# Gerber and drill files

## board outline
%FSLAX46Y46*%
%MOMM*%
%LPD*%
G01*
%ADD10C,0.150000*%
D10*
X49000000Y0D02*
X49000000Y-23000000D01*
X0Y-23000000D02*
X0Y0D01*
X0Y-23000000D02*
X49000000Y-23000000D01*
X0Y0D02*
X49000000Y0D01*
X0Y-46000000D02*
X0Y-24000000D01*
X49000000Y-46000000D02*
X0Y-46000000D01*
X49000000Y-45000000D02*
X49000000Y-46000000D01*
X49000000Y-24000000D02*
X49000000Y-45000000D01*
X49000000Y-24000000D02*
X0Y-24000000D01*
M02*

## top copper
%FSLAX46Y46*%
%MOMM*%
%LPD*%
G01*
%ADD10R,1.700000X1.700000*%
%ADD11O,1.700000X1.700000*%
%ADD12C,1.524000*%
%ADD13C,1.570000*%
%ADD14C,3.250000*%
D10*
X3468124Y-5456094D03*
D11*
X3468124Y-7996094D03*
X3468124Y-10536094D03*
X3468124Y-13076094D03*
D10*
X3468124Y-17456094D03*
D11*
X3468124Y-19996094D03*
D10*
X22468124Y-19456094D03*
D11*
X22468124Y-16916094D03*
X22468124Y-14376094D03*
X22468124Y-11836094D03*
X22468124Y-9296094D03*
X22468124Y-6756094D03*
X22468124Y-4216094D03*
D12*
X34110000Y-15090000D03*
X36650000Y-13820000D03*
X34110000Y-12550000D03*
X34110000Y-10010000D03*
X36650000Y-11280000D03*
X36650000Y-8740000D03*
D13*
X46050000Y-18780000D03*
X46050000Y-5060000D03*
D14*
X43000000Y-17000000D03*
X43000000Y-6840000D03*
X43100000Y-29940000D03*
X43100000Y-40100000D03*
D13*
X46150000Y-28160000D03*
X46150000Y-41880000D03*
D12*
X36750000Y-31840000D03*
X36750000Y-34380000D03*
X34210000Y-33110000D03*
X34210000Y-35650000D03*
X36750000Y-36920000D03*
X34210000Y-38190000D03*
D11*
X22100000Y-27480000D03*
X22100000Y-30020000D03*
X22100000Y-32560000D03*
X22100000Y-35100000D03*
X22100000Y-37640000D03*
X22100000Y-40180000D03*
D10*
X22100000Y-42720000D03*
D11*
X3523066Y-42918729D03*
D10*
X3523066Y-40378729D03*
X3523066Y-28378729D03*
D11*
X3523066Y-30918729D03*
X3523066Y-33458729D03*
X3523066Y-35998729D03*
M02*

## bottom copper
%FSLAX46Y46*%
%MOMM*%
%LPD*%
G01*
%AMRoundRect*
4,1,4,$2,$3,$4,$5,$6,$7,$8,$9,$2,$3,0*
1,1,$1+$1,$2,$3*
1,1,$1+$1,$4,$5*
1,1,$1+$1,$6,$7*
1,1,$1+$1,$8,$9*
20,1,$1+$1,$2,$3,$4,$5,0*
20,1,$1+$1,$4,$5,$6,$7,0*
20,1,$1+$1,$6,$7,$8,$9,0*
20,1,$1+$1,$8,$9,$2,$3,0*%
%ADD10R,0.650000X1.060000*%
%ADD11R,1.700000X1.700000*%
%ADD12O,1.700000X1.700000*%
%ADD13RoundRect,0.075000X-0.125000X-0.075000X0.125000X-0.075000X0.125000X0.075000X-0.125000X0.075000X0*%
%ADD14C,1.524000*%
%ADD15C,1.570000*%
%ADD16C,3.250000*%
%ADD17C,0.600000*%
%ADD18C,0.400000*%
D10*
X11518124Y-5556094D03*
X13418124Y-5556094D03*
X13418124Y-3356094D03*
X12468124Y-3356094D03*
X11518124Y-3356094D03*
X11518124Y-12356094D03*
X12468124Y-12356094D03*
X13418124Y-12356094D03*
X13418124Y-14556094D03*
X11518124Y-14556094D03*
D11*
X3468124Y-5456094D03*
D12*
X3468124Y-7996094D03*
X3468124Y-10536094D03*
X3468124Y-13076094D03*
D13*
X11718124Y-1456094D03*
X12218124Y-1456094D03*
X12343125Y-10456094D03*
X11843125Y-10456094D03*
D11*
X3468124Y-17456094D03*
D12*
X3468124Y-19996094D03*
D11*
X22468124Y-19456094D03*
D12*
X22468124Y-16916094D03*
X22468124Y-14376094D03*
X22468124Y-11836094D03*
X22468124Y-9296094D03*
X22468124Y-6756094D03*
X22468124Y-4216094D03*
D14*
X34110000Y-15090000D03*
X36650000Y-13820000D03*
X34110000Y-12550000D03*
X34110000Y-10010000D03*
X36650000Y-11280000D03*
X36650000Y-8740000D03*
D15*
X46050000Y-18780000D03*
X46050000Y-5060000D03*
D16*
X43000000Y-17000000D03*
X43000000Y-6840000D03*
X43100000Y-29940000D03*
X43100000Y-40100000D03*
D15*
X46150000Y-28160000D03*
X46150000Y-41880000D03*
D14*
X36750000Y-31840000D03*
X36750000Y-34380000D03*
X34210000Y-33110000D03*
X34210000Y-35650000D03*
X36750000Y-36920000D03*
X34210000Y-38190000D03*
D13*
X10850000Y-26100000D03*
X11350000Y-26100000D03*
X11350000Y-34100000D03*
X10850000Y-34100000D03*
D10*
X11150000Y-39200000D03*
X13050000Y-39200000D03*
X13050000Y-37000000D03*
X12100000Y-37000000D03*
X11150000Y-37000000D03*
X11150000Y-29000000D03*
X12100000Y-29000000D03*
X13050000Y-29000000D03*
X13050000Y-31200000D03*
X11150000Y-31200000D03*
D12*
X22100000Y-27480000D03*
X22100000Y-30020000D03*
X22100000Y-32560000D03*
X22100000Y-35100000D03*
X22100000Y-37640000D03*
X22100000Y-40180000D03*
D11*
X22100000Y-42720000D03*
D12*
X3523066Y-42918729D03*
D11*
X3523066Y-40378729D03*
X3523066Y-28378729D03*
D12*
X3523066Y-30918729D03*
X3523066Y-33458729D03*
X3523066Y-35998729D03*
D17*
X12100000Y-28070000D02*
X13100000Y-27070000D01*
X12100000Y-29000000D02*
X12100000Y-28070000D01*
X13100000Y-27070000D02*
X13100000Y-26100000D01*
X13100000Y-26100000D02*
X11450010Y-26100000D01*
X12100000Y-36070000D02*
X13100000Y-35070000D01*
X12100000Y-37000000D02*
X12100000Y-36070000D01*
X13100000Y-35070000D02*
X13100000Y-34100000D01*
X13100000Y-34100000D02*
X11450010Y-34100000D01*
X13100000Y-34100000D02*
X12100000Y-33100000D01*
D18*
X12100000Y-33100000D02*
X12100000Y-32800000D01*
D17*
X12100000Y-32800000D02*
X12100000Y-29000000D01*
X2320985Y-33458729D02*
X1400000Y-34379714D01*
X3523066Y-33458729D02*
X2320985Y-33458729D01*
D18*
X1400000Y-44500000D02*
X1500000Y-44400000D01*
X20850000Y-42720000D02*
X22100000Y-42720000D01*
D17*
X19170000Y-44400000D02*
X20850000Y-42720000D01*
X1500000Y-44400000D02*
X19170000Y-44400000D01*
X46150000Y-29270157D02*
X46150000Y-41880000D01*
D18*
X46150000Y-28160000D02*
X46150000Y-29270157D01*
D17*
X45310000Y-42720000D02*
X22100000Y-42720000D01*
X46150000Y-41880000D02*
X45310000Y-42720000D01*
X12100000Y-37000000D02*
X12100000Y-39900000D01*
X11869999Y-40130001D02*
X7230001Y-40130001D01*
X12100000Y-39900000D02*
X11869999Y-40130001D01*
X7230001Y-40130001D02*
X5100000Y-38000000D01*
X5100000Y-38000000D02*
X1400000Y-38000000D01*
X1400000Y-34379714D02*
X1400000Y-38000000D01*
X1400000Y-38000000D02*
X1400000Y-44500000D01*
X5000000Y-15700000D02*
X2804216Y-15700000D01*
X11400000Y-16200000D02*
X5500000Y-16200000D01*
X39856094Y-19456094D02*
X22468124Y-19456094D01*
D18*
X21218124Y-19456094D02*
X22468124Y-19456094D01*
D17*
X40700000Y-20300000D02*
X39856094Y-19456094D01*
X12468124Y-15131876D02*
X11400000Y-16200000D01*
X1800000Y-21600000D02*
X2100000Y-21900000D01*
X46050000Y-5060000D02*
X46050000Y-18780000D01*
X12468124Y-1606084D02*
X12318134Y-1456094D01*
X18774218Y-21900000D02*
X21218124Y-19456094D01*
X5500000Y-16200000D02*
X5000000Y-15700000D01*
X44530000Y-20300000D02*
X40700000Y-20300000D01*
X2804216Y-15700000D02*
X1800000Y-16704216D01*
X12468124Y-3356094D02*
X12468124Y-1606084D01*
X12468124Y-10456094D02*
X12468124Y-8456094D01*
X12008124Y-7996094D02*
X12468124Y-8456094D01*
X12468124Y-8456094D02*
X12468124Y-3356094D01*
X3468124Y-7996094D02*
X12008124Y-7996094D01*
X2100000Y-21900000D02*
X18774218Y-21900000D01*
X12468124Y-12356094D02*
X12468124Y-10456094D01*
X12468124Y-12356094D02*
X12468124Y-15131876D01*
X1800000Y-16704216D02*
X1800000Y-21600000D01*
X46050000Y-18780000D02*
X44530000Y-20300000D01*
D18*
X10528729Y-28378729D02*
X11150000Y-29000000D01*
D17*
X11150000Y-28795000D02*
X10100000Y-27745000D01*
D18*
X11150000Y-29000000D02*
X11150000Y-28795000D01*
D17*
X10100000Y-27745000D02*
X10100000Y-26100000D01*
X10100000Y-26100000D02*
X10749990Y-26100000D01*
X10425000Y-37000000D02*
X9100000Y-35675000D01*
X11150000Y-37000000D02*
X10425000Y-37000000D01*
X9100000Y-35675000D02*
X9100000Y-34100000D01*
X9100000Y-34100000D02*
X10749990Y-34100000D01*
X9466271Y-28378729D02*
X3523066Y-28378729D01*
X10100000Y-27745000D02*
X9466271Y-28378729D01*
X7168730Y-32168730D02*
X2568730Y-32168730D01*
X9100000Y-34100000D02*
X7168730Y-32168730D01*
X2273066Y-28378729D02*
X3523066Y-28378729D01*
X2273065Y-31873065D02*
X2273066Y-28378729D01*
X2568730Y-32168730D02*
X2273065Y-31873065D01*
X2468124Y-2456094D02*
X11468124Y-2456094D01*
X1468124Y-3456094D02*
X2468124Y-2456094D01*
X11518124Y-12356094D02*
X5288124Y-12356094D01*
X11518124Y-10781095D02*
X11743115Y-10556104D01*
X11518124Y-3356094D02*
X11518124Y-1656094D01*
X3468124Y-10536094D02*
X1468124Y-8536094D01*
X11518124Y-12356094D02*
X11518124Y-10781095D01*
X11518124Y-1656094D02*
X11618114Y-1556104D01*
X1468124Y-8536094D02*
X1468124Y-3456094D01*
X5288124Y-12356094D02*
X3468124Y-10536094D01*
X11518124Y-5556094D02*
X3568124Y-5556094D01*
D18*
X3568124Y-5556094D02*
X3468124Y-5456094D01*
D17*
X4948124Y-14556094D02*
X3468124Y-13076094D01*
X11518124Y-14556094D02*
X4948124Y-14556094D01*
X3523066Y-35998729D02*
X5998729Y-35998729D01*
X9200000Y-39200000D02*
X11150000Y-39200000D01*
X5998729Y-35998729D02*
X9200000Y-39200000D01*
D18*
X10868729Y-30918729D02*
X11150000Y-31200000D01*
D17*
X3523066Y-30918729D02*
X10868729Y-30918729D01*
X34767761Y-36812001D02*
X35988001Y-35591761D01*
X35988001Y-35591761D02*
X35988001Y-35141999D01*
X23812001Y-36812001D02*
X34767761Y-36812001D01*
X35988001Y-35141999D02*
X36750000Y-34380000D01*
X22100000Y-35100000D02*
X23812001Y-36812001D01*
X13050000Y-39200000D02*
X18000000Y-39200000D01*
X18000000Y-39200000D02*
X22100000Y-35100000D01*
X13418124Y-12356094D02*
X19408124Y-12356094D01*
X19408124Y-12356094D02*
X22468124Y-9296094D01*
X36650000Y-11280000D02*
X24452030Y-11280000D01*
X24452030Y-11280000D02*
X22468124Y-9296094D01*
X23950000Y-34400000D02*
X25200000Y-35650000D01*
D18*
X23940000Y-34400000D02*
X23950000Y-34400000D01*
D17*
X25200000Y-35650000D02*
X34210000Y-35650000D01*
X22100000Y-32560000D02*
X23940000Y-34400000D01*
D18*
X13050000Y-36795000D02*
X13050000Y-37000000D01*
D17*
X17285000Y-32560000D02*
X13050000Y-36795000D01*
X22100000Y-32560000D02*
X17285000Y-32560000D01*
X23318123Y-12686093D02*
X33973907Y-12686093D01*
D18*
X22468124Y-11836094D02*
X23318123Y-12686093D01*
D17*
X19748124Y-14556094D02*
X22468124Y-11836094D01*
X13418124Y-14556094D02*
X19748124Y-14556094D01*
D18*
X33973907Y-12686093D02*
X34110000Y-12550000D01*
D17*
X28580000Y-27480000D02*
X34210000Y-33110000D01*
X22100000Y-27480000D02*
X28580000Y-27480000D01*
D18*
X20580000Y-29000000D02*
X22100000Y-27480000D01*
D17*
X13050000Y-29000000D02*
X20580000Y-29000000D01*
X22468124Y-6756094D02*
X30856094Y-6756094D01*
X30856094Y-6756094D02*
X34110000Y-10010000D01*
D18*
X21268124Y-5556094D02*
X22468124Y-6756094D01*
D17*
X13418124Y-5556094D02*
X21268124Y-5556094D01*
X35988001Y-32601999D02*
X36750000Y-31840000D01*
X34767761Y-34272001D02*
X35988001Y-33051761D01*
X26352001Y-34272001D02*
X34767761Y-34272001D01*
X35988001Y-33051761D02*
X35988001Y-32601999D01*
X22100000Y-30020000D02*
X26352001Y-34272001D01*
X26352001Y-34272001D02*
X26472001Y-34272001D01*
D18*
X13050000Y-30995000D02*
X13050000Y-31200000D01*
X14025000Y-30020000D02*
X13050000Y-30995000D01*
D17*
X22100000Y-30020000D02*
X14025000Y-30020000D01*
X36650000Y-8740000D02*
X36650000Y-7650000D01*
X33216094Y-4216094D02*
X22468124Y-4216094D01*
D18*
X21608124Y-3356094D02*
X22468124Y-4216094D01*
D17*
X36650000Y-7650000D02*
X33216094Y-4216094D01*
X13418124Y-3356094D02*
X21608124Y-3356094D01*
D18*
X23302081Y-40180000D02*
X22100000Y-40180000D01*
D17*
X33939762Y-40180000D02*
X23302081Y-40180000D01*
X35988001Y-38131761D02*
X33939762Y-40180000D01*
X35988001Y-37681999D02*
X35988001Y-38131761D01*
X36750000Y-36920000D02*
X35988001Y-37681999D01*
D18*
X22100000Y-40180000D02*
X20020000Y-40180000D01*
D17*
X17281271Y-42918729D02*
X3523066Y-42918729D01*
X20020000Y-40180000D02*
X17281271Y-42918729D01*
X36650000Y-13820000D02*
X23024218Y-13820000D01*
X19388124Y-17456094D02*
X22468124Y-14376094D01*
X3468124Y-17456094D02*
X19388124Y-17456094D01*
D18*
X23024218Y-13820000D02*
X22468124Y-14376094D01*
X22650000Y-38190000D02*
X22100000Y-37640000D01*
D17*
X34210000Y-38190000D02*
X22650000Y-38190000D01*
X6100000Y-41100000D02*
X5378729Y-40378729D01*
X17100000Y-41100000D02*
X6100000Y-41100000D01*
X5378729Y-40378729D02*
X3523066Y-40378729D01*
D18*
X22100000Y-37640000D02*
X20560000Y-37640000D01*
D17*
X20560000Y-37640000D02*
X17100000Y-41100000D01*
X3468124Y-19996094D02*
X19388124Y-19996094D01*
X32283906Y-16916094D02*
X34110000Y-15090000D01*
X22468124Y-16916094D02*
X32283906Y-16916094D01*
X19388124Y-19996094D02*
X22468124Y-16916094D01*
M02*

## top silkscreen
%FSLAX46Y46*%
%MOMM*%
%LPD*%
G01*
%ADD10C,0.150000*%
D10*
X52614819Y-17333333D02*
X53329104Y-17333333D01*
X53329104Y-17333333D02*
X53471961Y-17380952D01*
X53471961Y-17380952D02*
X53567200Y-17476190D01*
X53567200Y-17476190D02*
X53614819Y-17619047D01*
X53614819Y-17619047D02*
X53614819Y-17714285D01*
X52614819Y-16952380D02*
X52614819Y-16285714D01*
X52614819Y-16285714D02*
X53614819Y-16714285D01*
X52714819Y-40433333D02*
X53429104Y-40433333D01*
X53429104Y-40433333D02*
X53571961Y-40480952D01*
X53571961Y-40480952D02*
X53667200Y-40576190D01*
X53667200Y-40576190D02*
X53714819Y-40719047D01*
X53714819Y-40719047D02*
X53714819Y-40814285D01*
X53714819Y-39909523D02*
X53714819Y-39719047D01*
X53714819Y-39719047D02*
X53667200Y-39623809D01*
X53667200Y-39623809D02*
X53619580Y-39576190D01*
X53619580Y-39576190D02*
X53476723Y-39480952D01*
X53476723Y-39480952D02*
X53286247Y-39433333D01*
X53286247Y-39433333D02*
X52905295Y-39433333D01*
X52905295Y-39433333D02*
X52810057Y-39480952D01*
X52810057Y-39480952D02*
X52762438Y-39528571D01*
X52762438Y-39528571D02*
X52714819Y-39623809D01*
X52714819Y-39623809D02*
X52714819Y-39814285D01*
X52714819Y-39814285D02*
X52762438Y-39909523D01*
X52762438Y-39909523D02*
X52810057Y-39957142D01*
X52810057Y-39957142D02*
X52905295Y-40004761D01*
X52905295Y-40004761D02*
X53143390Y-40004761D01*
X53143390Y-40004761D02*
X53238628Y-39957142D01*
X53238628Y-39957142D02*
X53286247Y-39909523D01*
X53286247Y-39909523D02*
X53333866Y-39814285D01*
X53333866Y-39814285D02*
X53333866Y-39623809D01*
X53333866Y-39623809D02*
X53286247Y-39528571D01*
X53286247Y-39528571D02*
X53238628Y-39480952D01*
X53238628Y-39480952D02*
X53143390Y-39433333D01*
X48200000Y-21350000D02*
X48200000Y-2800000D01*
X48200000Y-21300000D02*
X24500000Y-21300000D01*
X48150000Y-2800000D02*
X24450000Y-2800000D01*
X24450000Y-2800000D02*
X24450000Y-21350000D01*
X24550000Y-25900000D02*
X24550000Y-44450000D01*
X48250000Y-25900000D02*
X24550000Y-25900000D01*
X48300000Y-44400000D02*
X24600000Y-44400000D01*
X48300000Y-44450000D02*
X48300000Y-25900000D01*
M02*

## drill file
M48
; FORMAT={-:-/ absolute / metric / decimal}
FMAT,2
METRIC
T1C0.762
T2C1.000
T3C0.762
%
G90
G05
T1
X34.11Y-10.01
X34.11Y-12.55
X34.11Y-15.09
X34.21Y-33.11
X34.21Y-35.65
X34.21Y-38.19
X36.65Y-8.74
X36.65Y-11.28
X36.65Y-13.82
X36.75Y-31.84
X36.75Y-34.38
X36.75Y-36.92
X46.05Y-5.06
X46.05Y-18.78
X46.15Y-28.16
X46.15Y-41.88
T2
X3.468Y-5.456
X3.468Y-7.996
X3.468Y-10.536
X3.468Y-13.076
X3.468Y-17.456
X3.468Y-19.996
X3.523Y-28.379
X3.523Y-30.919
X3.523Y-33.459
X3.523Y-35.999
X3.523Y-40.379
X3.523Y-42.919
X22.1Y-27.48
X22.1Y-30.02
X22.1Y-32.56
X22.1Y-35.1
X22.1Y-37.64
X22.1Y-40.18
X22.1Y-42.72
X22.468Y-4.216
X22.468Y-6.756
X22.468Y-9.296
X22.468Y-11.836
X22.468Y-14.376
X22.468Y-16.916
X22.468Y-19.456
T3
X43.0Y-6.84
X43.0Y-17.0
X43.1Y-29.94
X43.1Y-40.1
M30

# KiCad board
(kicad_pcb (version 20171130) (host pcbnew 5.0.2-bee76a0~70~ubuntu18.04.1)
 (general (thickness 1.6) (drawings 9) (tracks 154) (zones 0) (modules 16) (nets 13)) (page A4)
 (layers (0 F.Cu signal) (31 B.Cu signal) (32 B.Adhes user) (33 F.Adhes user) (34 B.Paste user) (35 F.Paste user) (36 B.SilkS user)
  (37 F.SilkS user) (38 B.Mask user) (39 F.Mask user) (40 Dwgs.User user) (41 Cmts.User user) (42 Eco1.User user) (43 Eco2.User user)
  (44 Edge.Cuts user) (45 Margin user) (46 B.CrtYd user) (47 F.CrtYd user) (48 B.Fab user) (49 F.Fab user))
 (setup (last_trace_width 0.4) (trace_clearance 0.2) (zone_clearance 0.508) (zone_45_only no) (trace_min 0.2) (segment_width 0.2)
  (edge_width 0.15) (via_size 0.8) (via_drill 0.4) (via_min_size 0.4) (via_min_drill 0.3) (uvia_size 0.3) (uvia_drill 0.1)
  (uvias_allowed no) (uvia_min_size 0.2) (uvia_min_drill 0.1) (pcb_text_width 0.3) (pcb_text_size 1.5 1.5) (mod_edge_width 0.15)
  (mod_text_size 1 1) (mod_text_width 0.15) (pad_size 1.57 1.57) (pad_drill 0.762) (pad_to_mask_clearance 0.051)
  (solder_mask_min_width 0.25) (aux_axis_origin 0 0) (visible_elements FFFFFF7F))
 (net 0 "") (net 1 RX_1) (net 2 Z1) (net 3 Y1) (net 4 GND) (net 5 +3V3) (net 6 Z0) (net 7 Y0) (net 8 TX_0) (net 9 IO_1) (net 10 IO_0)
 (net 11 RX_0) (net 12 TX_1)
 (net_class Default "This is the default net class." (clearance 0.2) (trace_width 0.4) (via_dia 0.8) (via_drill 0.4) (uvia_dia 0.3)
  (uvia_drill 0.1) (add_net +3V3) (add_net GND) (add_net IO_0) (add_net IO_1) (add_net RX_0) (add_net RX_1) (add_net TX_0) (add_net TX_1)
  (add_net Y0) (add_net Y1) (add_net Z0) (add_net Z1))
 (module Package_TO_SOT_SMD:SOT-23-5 (layer B.Cu) (at 12.468124 4.456094 270)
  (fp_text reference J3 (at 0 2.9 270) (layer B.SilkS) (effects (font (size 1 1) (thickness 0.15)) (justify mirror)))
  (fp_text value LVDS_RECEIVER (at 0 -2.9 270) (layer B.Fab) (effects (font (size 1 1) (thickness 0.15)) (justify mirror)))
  (pad 5 smd rect (at 1.1 0.95 270) (size 1.06 0.65) (layers B.Cu B.Paste B.Mask) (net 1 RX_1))
  (pad 4 smd rect (at 1.1 -0.95 270) (size 1.06 0.65) (layers B.Cu B.Paste B.Mask) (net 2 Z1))
  (pad 3 smd rect (at -1.1 -0.95 270) (size 1.06 0.65) (layers B.Cu B.Paste B.Mask) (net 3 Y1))
  (pad 2 smd rect (at -1.1 0 270) (size 1.06 0.65) (layers B.Cu B.Paste B.Mask) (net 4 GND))
  (pad 1 smd rect (at -1.1 0.95 270) (size 1.06 0.65) (layers B.Cu B.Paste B.Mask) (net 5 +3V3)))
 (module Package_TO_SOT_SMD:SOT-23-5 (layer B.Cu) (at 12.468124 13.456094 270)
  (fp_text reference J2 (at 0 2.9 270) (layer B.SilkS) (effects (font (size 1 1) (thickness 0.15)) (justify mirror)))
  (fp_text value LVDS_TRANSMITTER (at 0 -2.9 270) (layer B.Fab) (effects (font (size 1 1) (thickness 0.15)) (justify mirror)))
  (pad 1 smd rect (at -1.1 0.95 270) (size 1.06 0.65) (layers B.Cu B.Paste B.Mask) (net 5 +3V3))
  (pad 2 smd rect (at -1.1 0 270) (size 1.06 0.65) (layers B.Cu B.Paste B.Mask) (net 4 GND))
  (pad 3 smd rect (at -1.1 -0.95 270) (size 1.06 0.65) (layers B.Cu B.Paste B.Mask) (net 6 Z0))
  (pad 4 smd rect (at 1.1 -0.95 270) (size 1.06 0.65) (layers B.Cu B.Paste B.Mask) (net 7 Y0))
  (pad 5 smd rect (at 1.1 0.95 270) (size 1.06 0.65) (layers B.Cu B.Paste B.Mask) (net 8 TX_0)))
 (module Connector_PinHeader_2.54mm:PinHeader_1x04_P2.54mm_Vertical (layer B.Cu) (at 3.468124 5.456094 180)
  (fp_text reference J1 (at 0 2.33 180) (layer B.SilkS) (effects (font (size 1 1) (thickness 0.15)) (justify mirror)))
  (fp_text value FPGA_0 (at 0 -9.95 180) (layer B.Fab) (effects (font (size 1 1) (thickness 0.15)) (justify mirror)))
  (pad 1 thru_hole rect (at 0 0 180) (size 1.7 1.7) (drill 1) (layers *.Cu *.Mask) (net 1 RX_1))
  (pad 2 thru_hole oval (at 0 -2.54 180) (size 1.7 1.7) (drill 1) (layers *.Cu *.Mask) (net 4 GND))
  (pad 3 thru_hole oval (at 0 -5.08 180) (size 1.7 1.7) (drill 1) (layers *.Cu *.Mask) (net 5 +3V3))
  (pad 4 thru_hole oval (at 0 -7.62 180) (size 1.7 1.7) (drill 1) (layers *.Cu *.Mask) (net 8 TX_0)))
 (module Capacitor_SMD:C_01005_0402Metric (layer B.Cu) (at 11.968124 1.456094)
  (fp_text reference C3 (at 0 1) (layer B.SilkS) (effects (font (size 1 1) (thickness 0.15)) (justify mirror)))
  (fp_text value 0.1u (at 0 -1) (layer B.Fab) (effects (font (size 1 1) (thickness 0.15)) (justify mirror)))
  (pad "" smd roundrect (at -0.275 0) (size 0.27 0.27) (layers B.Paste) (roundrect_rratio 0.25))
  (pad "" smd roundrect (at 0.275 0) (size 0.27 0.27) (layers B.Paste) (roundrect_rratio 0.25))
  (pad 1 smd roundrect (at -0.25 0) (size 0.4 0.3) (layers B.Cu B.Mask) (roundrect_rratio 0.25) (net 5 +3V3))
  (pad 2 smd roundrect (at 0.25 0) (size 0.4 0.3) (layers B.Cu B.Mask) (roundrect_rratio 0.25) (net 4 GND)))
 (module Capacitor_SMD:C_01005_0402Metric (layer B.Cu) (at 12.093125 10.456094)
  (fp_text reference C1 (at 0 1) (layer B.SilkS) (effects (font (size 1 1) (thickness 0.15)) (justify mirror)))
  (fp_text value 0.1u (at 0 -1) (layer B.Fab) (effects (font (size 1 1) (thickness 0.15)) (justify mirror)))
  (pad 2 smd roundrect (at 0.25 0) (size 0.4 0.3) (layers B.Cu B.Mask) (roundrect_rratio 0.25) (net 4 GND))
  (pad 1 smd roundrect (at -0.25 0) (size 0.4 0.3) (layers B.Cu B.Mask) (roundrect_rratio 0.25) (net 5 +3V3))
  (pad "" smd roundrect (at 0.275 0) (size 0.27 0.27) (layers B.Paste) (roundrect_rratio 0.25))
  (pad "" smd roundrect (at -0.275 0) (size 0.27 0.27) (layers B.Paste) (roundrect_rratio 0.25)))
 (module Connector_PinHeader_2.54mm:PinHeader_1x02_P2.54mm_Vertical (layer B.Cu) (at 3.468124 17.456094 180)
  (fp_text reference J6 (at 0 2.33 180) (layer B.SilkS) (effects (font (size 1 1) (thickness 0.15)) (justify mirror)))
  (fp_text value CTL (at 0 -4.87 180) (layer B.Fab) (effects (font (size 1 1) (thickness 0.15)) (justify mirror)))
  (pad 1 thru_hole rect (at 0 0 180) (size 1.7 1.7) (drill 1) (layers *.Cu *.Mask) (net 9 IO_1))
  (pad 2 thru_hole oval (at 0 -2.54 180) (size 1.7 1.7) (drill 1) (layers *.Cu *.Mask) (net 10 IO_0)))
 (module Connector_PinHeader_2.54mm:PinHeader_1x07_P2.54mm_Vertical (layer B.Cu) (at 22.468124 19.456094)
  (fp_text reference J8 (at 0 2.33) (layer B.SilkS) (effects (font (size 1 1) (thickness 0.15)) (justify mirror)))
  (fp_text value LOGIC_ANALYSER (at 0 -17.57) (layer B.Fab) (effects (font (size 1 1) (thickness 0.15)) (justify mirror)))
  (pad 1 thru_hole rect (at 0 0) (size 1.7 1.7) (drill 1) (layers *.Cu *.Mask) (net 4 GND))
  (pad 2 thru_hole oval (at 0 -2.54) (size 1.7 1.7) (drill 1) (layers *.Cu *.Mask) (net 10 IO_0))
  (pad 3 thru_hole oval (at 0 -5.08) (size 1.7 1.7) (drill 1) (layers *.Cu *.Mask) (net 9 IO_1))
  (pad 4 thru_hole oval (at 0 -7.62) (size 1.7 1.7) (drill 1) (layers *.Cu *.Mask) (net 7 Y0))
  (pad 5 thru_hole oval (at 0 -10.16) (size 1.7 1.7) (drill 1) (layers *.Cu *.Mask) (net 6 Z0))
  (pad 6 thru_hole oval (at 0 -12.7) (size 1.7 1.7) (drill 1) (layers *.Cu *.Mask) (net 2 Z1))
  (pad 7 thru_hole oval (at 0 -15.24) (size 1.7 1.7) (drill 1) (layers *.Cu *.Mask) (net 3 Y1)))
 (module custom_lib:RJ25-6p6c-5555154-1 (layer F.Cu) (at 43 17 90)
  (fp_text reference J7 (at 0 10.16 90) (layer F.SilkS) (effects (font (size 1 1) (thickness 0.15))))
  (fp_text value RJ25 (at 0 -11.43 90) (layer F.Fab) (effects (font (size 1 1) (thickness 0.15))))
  (fp_line (start -4.35 5.2) (end 14.2 5.2) (layer F.SilkS) (width 0.15))
  (fp_line (start -4.3 5.2) (end -4.3 -18.5) (layer F.SilkS) (width 0.15))
  (fp_line (start 14.2 5.15) (end 14.2 -18.55) (layer F.SilkS) (width 0.15))
  (fp_line (start 14.2 -18.55) (end -4.35 -18.55) (layer F.SilkS) (width 0.15))
  (pad 1 thru_hole circle (at 1.91 -8.89 90) (size 1.524 1.524) (drill 0.762) (layers *.Cu *.Mask) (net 10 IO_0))
  (pad 2 thru_hole circle (at 3.18 -6.35 90) (size 1.524 1.524) (drill 0.762) (layers *.Cu *.Mask) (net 9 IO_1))
  (pad 3 thru_hole circle (at 4.45 -8.89 90) (size 1.524 1.524) (drill 0.762) (layers *.Cu *.Mask) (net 7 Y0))
  (pad 4 thru_hole circle (at 6.99 -8.89 90) (size 1.524 1.524) (drill 0.762) (layers *.Cu *.Mask) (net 2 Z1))
  (pad 5 thru_hole circle (at 5.72 -6.35 90) (size 1.524 1.524) (drill 0.762) (layers *.Cu *.Mask) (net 6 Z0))
  (pad 6 thru_hole circle (at 8.26 -6.35 90) (size 1.524 1.524) (drill 0.762) (layers *.Cu *.Mask) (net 3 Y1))
  (pad 7 thru_hole circle (at -1.78 3.05 90) (size 1.57 1.57) (drill 0.762) (layers *.Cu *.Mask) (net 4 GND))
  (pad 8 thru_hole circle (at 11.94 3.05 90) (size 1.57 1.57) (drill 0.762) (layers *.Cu *.Mask) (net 4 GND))
  (pad "" np_thru_hole circle (at 0 0 90) (size 3.25 3.25) (drill 0.762) (layers *.Cu *.Mask))
  (pad "" np_thru_hole circle (at 10.16 0 90) (size 3.25 3.25) (drill 0.762) (layers *.Cu *.Mask)))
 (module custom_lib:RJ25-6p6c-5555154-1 (layer F.Cu) (at 43.1 40.1 90)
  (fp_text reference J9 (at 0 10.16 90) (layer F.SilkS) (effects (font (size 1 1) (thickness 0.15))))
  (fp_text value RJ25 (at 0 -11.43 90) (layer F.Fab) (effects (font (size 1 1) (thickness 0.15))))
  (fp_line (start 14.2 -18.55) (end -4.35 -18.55) (layer F.SilkS) (width 0.15))
  (fp_line (start 14.2 5.15) (end 14.2 -18.55) (layer F.SilkS) (width 0.15))
  (fp_line (start -4.3 5.2) (end -4.3 -18.5) (layer F.SilkS) (width 0.15))
  (fp_line (start -4.35 5.2) (end 14.2 5.2) (layer F.SilkS) (width 0.15))
  (pad "" np_thru_hole circle (at 10.16 0 90) (size 3.25 3.25) (drill 0.762) (layers *.Cu *.Mask))
  (pad "" np_thru_hole circle (at 0 0 90) (size 3.25 3.25) (drill 0.762) (layers *.Cu *.Mask))
  (pad 8 thru_hole circle (at 11.94 3.05 90) (size 1.57 1.57) (drill 0.762) (layers *.Cu *.Mask) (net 4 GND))
  (pad 7 thru_hole circle (at -1.78 3.05 90) (size 1.57 1.57) (drill 0.762) (layers *.Cu *.Mask) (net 4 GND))
  (pad 6 thru_hole circle (at 8.26 -6.35 90) (size 1.524 1.524) (drill 0.762) (layers *.Cu *.Mask) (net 3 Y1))
  (pad 5 thru_hole circle (at 5.72 -6.35 90) (size 1.524 1.524) (drill 0.762) (layers *.Cu *.Mask) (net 6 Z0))
  (pad 4 thru_hole circle (at 6.99 -8.89 90) (size 1.524 1.524) (drill 0.762) (layers *.Cu *.Mask) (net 2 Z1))
  (pad 3 thru_hole circle (at 4.45 -8.89 90) (size 1.524 1.524) (drill 0.762) (layers *.Cu *.Mask) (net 7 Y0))
  (pad 2 thru_hole circle (at 3.18 -6.35 90) (size 1.524 1.524) (drill 0.762) (layers *.Cu *.Mask) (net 9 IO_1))
  (pad 1 thru_hole circle (at 1.91 -8.89 90) (size 1.524 1.524) (drill 0.762) (layers *.Cu *.Mask) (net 10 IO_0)))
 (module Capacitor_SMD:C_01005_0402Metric (layer B.Cu) (at 11.1 26.1)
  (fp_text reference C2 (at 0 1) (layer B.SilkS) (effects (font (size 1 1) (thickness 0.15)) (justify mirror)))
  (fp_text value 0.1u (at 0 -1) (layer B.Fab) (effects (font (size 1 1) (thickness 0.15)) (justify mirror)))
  (pad "" smd roundrect (at -0.275 0) (size 0.27 0.27) (layers B.Paste) (roundrect_rratio 0.25))
  (pad "" smd roundrect (at 0.275 0) (size 0.27 0.27) (layers B.Paste) (roundrect_rratio 0.25))
  (pad 1 smd roundrect (at -0.25 0) (size 0.4 0.3) (layers B.Cu B.Mask) (roundrect_rratio 0.25) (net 5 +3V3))
  (pad 2 smd roundrect (at 0.25 0) (size 0.4 0.3) (layers B.Cu B.Mask) (roundrect_rratio 0.25) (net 4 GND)))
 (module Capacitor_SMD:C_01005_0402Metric (layer B.Cu) (at 11.1 34.1)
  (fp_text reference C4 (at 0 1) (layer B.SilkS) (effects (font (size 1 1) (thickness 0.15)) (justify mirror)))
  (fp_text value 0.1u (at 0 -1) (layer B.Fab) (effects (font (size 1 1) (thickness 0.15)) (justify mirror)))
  (pad 2 smd roundrect (at 0.25 0) (size 0.4 0.3) (layers B.Cu B.Mask) (roundrect_rratio 0.25) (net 4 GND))
  (pad 1 smd roundrect (at -0.25 0) (size 0.4 0.3) (layers B.Cu B.Mask) (roundrect_rratio 0.25) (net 5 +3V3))
  (pad "" smd roundrect (at 0.275 0) (size 0.27 0.27) (layers B.Paste) (roundrect_rratio 0.25))
  (pad "" smd roundrect (at -0.275 0) (size 0.27 0.27) (layers B.Paste) (roundrect_rratio 0.25)))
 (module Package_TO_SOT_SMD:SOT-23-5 (layer B.Cu) (at 12.1 38.1 270)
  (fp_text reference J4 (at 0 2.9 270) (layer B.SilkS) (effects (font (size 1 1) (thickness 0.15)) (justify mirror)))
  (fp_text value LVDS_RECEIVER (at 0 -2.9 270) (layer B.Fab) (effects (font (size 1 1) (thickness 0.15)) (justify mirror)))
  (pad 5 smd rect (at 1.1 0.95 270) (size 1.06 0.65) (layers B.Cu B.Paste B.Mask) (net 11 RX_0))
  (pad 4 smd rect (at 1.1 -0.95 270) (size 1.06 0.65) (layers B.Cu B.Paste B.Mask) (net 6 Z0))
  (pad 3 smd rect (at -1.1 -0.95 270) (size 1.06 0.65) (layers B.Cu B.Paste B.Mask) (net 7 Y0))
  (pad 2 smd rect (at -1.1 0 270) (size 1.06 0.65) (layers B.Cu B.Paste B.Mask) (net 4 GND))
  (pad 1 smd rect (at -1.1 0.95 270) (size 1.06 0.65) (layers B.Cu B.Paste B.Mask) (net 5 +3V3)))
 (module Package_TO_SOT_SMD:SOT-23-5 (layer B.Cu) (at 12.1 30.1 270)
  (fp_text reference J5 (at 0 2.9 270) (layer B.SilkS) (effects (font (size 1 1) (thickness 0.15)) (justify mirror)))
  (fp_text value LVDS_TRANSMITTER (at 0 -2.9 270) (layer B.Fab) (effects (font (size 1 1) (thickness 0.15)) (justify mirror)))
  (pad 1 smd rect (at -1.1 0.95 270) (size 1.06 0.65) (layers B.Cu B.Paste B.Mask) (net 5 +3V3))
  (pad 2 smd rect (at -1.1 0 270) (size 1.06 0.65) (layers B.Cu B.Paste B.Mask) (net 4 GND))
  (pad 3 smd rect (at -1.1 -0.95 270) (size 1.06 0.65) (layers B.Cu B.Paste B.Mask) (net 2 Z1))
  (pad 4 smd rect (at 1.1 -0.95 270) (size 1.06 0.65) (layers B.Cu B.Paste B.Mask) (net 3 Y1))
  (pad 5 smd rect (at 1.1 0.95 270) (size 1.06 0.65) (layers B.Cu B.Paste B.Mask) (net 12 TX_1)))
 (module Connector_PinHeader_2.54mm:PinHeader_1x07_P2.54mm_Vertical (layer B.Cu) (at 22.1 42.72)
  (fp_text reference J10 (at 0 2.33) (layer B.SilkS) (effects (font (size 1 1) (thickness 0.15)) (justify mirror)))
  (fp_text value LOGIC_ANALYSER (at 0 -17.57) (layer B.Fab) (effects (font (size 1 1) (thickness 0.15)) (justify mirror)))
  (pad 7 thru_hole oval (at 0 -15.24) (size 1.7 1.7) (drill 1) (layers *.Cu *.Mask) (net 2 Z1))
  (pad 6 thru_hole oval (at 0 -12.7) (size 1.7 1.7) (drill 1) (layers *.Cu *.Mask) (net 3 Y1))
  (pad 5 thru_hole oval (at 0 -10.16) (size 1.7 1.7) (drill 1) (layers *.Cu *.Mask) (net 7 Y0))
  (pad 4 thru_hole oval (at 0 -7.62) (size 1.7 1.7) (drill 1) (layers *.Cu *.Mask) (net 6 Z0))
  (pad 3 thru_hole oval (at 0 -5.08) (size 1.7 1.7) (drill 1) (layers *.Cu *.Mask) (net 10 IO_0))
  (pad 2 thru_hole oval (at 0 -2.54) (size 1.7 1.7) (drill 1) (layers *.Cu *.Mask) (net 9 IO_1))
  (pad 1 thru_hole rect (at 0 0) (size 1.7 1.7) (drill 1) (layers *.Cu *.Mask) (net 4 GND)))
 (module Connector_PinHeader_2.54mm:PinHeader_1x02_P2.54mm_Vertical (layer B.Cu) (at 3.523066 40.378729 180)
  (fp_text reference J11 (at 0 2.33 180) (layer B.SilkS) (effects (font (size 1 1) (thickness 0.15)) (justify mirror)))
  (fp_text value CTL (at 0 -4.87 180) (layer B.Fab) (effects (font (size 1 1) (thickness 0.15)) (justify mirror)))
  (pad 2 thru_hole oval (at 0 -2.54 180) (size 1.7 1.7) (drill 1) (layers *.Cu *.Mask) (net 9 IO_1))
  (pad 1 thru_hole rect (at 0 0 180) (size 1.7 1.7) (drill 1) (layers *.Cu *.Mask) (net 10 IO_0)))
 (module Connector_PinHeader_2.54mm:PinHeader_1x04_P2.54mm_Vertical (layer B.Cu) (at 3.523066 28.378729 180)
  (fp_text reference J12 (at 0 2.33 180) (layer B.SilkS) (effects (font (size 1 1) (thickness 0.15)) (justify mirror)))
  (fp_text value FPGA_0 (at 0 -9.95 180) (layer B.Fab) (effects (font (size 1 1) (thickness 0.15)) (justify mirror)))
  (pad 1 thru_hole rect (at 0 0 180) (size 1.7 1.7) (drill 1) (layers *.Cu *.Mask) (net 5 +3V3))
  (pad 2 thru_hole oval (at 0 -2.54 180) (size 1.7 1.7) (drill 1) (layers *.Cu *.Mask) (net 12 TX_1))
  (pad 3 thru_hole oval (at 0 -5.08 180) (size 1.7 1.7) (drill 1) (layers *.Cu *.Mask) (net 4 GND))
  (pad 4 thru_hole oval (at 0 -7.62 180) (size 1.7 1.7) (drill 1) (layers *.Cu *.Mask) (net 11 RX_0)))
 (gr_line (start 49 0) (end 49 23) (layer Edge.Cuts) (width 0.15))
 (gr_line (start 0 23) (end 0 0) (layer Edge.Cuts) (width 0.15))
 (gr_line (start 0 23) (end 49 23) (layer Edge.Cuts) (width 0.15))
 (gr_line (start 0 0) (end 49 0) (layer Edge.Cuts) (width 0.15))
 (gr_line (start 0 46) (end 0 24) (layer Edge.Cuts) (width 0.15))
 (gr_line (start 49 46) (end 0 46) (layer Edge.Cuts) (width 0.15))
 (gr_line (start 49 45) (end 49 46) (layer Edge.Cuts) (width 0.15))
 (gr_line (start 49 24) (end 49 45) (layer Edge.Cuts) (width 0.15))
 (gr_line (start 49 24) (end 0 24) (layer Edge.Cuts) (width 0.15))
 (segment (start 12.1 28.07) (end 13.1 27.07) (width 0.6) (layer B.Cu) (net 4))
 (segment (start 12.1 29) (end 12.1 28.07) (width 0.6) (layer B.Cu) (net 4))
 (segment (start 13.1 27.07) (end 13.1 26.1) (width 0.6) (layer B.Cu) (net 4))
 (segment (start 13.1 26.1) (end 11.45001 26.1) (width 0.6) (layer B.Cu) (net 4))
 (segment (start 12.1 36.07) (end 13.1 35.07) (width 0.6) (layer B.Cu) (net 4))
 (segment (start 12.1 37) (end 12.1 36.07) (width 0.6) (layer B.Cu) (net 4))
 (segment (start 13.1 35.07) (end 13.1 34.1) (width 0.6) (layer B.Cu) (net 4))
 (segment (start 13.1 34.1) (end 11.45001 34.1) (width 0.6) (layer B.Cu) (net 4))
 (segment (start 13.1 34.1) (end 12.1 33.1) (width 0.6) (layer B.Cu) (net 4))
 (segment (start 12.1 33.1) (end 12.1 32.8) (width 0.4) (layer B.Cu) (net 4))
 (segment (start 12.1 32.8) (end 12.1 29) (width 0.6) (layer B.Cu) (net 4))
 (segment (start 2.320985 33.458729) (end 1.4 34.379714) (width 0.6) (layer B.Cu) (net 4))
 (segment (start 3.523066 33.458729) (end 2.320985 33.458729) (width 0.6) (layer B.Cu) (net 4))
 (segment (start 1.4 44.5) (end 1.5 44.4) (width 0.4) (layer B.Cu) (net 4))
 (segment (start 20.85 42.72) (end 22.1 42.72) (width 0.4) (layer B.Cu) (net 4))
 (segment (start 19.17 44.4) (end 20.85 42.72) (width 0.6) (layer B.Cu) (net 4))
 (segment (start 1.5 44.4) (end 19.17 44.4) (width 0.6) (layer B.Cu) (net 4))
 (segment (start 46.15 29.270157) (end 46.15 41.88) (width 0.6) (layer B.Cu) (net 4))
 (segment (start 46.15 28.16) (end 46.15 29.270157) (width 0.4) (layer B.Cu) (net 4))
 (segment (start 45.31 42.72) (end 22.1 42.72) (width 0.6) (layer B.Cu) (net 4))
 (segment (start 46.15 41.88) (end 45.31 42.72) (width 0.6) (layer B.Cu) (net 4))
 (segment (start 12.1 37) (end 12.1 39.9) (width 0.6) (layer B.Cu) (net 4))
 (segment (start 11.869999 40.130001) (end 7.230001 40.130001) (width 0.6) (layer B.Cu) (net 4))
 (segment (start 12.1 39.9) (end 11.869999 40.130001) (width 0.6) (layer B.Cu) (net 4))
 (segment (start 7.230001 40.130001) (end 5.1 38) (width 0.6) (layer B.Cu) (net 4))
 (segment (start 5.1 38) (end 1.4 38) (width 0.6) (layer B.Cu) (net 4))
 (segment (start 1.4 34.379714) (end 1.4 38) (width 0.6) (layer B.Cu) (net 4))
 (segment (start 1.4 38) (end 1.4 44.5) (width 0.6) (layer B.Cu) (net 4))
 (segment (start 5 15.7) (end 2.804216 15.7) (width 0.6) (layer B.Cu) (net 4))
 (segment (start 11.4 16.2) (end 5.5 16.2) (width 0.6) (layer B.Cu) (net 4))
 (segment (start 39.856094 19.456094) (end 22.468124 19.456094) (width 0.6) (layer B.Cu) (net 4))
 (segment (start 21.218124 19.456094) (end 22.468124 19.456094) (width 0.4) (layer B.Cu) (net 4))
 (segment (start 40.7 20.3) (end 39.856094 19.456094) (width 0.6) (layer B.Cu) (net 4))
 (segment (start 12.468124 15.131876) (end 11.4 16.2) (width 0.6) (layer B.Cu) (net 4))
 (segment (start 1.8 21.6) (end 2.1 21.9) (width 0.6) (layer B.Cu) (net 4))
 (segment (start 46.05 5.06) (end 46.05 18.78) (width 0.6) (layer B.Cu) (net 4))
 (segment (start 12.468124 1.606084) (end 12.318134 1.456094) (width 0.6) (layer B.Cu) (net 4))
 (segment (start 18.774218 21.9) (end 21.218124 19.456094) (width 0.6) (layer B.Cu) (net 4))
 (segment (start 5.5 16.2) (end 5 15.7) (width 0.6) (layer B.Cu) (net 4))
 (segment (start 44.53 20.3) (end 40.7 20.3) (width 0.6) (layer B.Cu) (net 4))
 (segment (start 2.804216 15.7) (end 1.8 16.704216) (width 0.6) (layer B.Cu) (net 4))
 (segment (start 12.468124 3.356094) (end 12.468124 1.606084) (width 0.6) (layer B.Cu) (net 4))
 (segment (start 12.468124 10.456094) (end 12.468124 8.456094) (width 0.6) (layer B.Cu) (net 4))
 (segment (start 12.008124 7.996094) (end 12.468124 8.456094) (width 0.6) (layer B.Cu) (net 4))
 (segment (start 12.468124 8.456094) (end 12.468124 3.356094) (width 0.6) (layer B.Cu) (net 4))
 (segment (start 3.468124 7.996094) (end 12.008124 7.996094) (width 0.6) (layer B.Cu) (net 4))
 (segment (start 2.1 21.9) (end 18.774218 21.9) (width 0.6) (layer B.Cu) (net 4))
 (segment (start 12.468124 12.356094) (end 12.468124 10.456094) (width 0.6) (layer B.Cu) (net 4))
 (segment (start 12.468124 12.356094) (end 12.468124 15.131876) (width 0.6) (layer B.Cu) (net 4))
 (segment (start 1.8 16.704216) (end 1.8 21.6) (width 0.6) (layer B.Cu) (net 4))
 (segment (start 46.05 18.78) (end 44.53 20.3) (width 0.6) (layer B.Cu) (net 4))
 (segment (start 10.528729 28.378729) (end 11.15 29) (width 0.4) (layer B.Cu) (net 5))
 (segment (start 11.15 28.795) (end 10.1 27.745) (width 0.6) (layer B.Cu) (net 5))
 (segment (start 11.15 29) (end 11.15 28.795) (width 0.4) (layer B.Cu) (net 5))
 (segment (start 10.1 27.745) (end 10.1 26.1) (width 0.6) (layer B.Cu) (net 5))
 (segment (start 10.1 26.1) (end 10.74999 26.1) (width 0.6) (layer B.Cu) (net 5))
 (segment (start 10.425 37) (end 9.1 35.675) (width 0.6) (layer B.Cu) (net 5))
 (segment (start 11.15 37) (end 10.425 37) (width 0.6) (layer B.Cu) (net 5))
 (segment (start 9.1 35.675) (end 9.1 34.1) (width 0.6) (layer B.Cu) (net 5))
 (segment (start 9.1 34.1) (end 10.74999 34.1) (width 0.6) (layer B.Cu) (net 5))
 (segment (start 9.466271 28.378729) (end 3.523066 28.378729) (width 0.6) (layer B.Cu) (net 5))
 (segment (start 10.1 27.745) (end 9.466271 28.378729) (width 0.6) (layer B.Cu) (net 5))
 (segment (start 7.16873 32.16873) (end 2.56873 32.16873) (width 0.6) (layer B.Cu) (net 5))
 (segment (start 9.1 34.1) (end 7.16873 32.16873) (width 0.6) (layer B.Cu) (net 5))
 (segment (start 2.273066 28.378729) (end 3.523066 28.378729) (width 0.6) (layer B.Cu) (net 5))
 (segment (start 2.273065 31.873065) (end 2.273066 28.378729) (width 0.6) (layer B.Cu) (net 5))
 (segment (start 2.56873 32.16873) (end 2.273065 31.873065) (width 0.6) (layer B.Cu) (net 5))
 (segment (start 2.468124 2.456094) (end 11.468124 2.456094) (width 0.6) (layer B.Cu) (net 5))
 (segment (start 1.468124 3.456094) (end 2.468124 2.456094) (width 0.6) (layer B.Cu) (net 5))
 (segment (start 11.518124 12.356094) (end 5.288124 12.356094) (width 0.6) (layer B.Cu) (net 5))
 (segment (start 11.518124 10.781095) (end 11.743115 10.556104) (width 0.6) (layer B.Cu) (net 5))
 (segment (start 11.518124 3.356094) (end 11.518124 1.656094) (width 0.6) (layer B.Cu) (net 5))
 (segment (start 3.468124 10.536094) (end 1.468124 8.536094) (width 0.6) (layer B.Cu) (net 5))
 (segment (start 11.518124 12.356094) (end 11.518124 10.781095) (width 0.6) (layer B.Cu) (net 5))
 (segment (start 11.518124 1.656094) (end 11.618114 1.556104) (width 0.6) (layer B.Cu) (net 5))
 (segment (start 1.468124 8.536094) (end 1.468124 3.456094) (width 0.6) (layer B.Cu) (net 5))
 (segment (start 5.288124 12.356094) (end 3.468124 10.536094) (width 0.6) (layer B.Cu) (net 5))
 (segment (start 11.518124 5.556094) (end 3.568124 5.556094) (width 0.6) (layer B.Cu) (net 1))
 (segment (start 3.568124 5.556094) (end 3.468124 5.456094) (width 0.4) (layer B.Cu) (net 1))
 (segment (start 4.948124 14.556094) (end 3.468124 13.076094) (width 0.6) (layer B.Cu) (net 8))
 (segment (start 11.518124 14.556094) (end 4.948124 14.556094) (width 0.6) (layer B.Cu) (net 8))
 (segment (start 3.523066 35.998729) (end 5.998729 35.998729) (width 0.6) (layer B.Cu) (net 11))
 (segment (start 9.2 39.2) (end 11.15 39.2) (width 0.6) (layer B.Cu) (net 11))
 (segment (start 5.998729 35.998729) (end 9.2 39.2) (width 0.6) (layer B.Cu) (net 11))
 (segment (start 10.868729 30.918729) (end 11.15 31.2) (width 0.4) (layer B.Cu) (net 12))
 (segment (start 3.523066 30.918729) (end 10.868729 30.918729) (width 0.6) (layer B.Cu) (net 12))
 (segment (start 34.767761 36.812001) (end 35.988001 35.591761) (width 0.6) (layer B.Cu) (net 6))
 (segment (start 35.988001 35.591761) (end 35.988001 35.141999) (width 0.6) (layer B.Cu) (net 6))
 (segment (start 23.812001 36.812001) (end 34.767761 36.812001) (width 0.6) (layer B.Cu) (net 6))
 (segment (start 35.988001 35.141999) (end 36.75 34.38) (width 0.6) (layer B.Cu) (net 6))
 (segment (start 22.1 35.1) (end 23.812001 36.812001) (width 0.6) (layer B.Cu) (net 6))
 (segment (start 13.05 39.2) (end 18 39.2) (width 0.6) (layer B.Cu) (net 6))
 (segment (start 18 39.2) (end 22.1 35.1) (width 0.6) (layer B.Cu) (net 6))
 (segment (start 13.418124 12.356094) (end 19.408124 12.356094) (width 0.6) (layer B.Cu) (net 6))
 (segment (start 19.408124 12.356094) (end 22.468124 9.296094) (width 0.6) (layer B.Cu) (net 6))
 (segment (start 36.65 11.28) (end 24.45203 11.28) (width 0.6) (layer B.Cu) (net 6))
 (segment (start 24.45203 11.28) (end 22.468124 9.296094) (width 0.6) (layer B.Cu) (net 6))
 (segment (start 23.95 34.4) (end 25.2 35.65) (width 0.6) (layer B.Cu) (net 7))
 (segment (start 23.94 34.4) (end 23.95 34.4) (width 0.4) (layer B.Cu) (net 7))
 (segment (start 25.2 35.65) (end 34.21 35.65) (width 0.6) (layer B.Cu) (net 7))
 (segment (start 22.1 32.56) (end 23.94 34.4) (width 0.6) (layer B.Cu) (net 7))
 (segment (start 13.05 36.795) (end 13.05 37) (width 0.4) (layer B.Cu) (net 7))
 (segment (start 17.285 32.56) (end 13.05 36.795) (width 0.6) (layer B.Cu) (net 7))
 (segment (start 22.1 32.56) (end 17.285 32.56) (width 0.6) (layer B.Cu) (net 7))
 (segment (start 23.318123 12.686093) (end 33.973907 12.686093) (width 0.6) (layer B.Cu) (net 7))
 (segment (start 22.468124 11.836094) (end 23.318123 12.686093) (width 0.4) (layer B.Cu) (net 7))
 (segment (start 19.748124 14.556094) (end 22.468124 11.836094) (width 0.6) (layer B.Cu) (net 7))
 (segment (start 13.418124 14.556094) (end 19.748124 14.556094) (width 0.6) (layer B.Cu) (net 7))
 (segment (start 33.973907 12.686093) (end 34.11 12.55) (width 0.4) (layer B.Cu) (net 7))
 (segment (start 28.58 27.48) (end 34.21 33.11) (width 0.6) (layer B.Cu) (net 2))
 (segment (start 22.1 27.48) (end 28.58 27.48) (width 0.6) (layer B.Cu) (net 2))
 (segment (start 20.58 29) (end 22.1 27.48) (width 0.4) (layer B.Cu) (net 2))
 (segment (start 13.05 29) (end 20.58 29) (width 0.6) (layer B.Cu) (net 2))
 (segment (start 22.468124 6.756094) (end 30.856094 6.756094) (width 0.6) (layer B.Cu) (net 2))
 (segment (start 30.856094 6.756094) (end 34.11 10.01) (width 0.6) (layer B.Cu) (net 2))
 (segment (start 21.268124 5.556094) (end 22.468124 6.756094) (width 0.4) (layer B.Cu) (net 2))
 (segment (start 13.418124 5.556094) (end 21.268124 5.556094) (width 0.6) (layer B.Cu) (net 2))
 (segment (start 35.988001 32.601999) (end 36.75 31.84) (width 0.6) (layer B.Cu) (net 3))
 (segment (start 34.767761 34.272001) (end 35.988001 33.051761) (width 0.6) (layer B.Cu) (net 3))
 (segment (start 26.352001 34.272001) (end 34.767761 34.272001) (width 0.6) (layer B.Cu) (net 3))
 (segment (start 35.988001 33.051761) (end 35.988001 32.601999) (width 0.6) (layer B.Cu) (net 3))
 (segment (start 22.1 30.02) (end 26.352001 34.272001) (width 0.6) (layer B.Cu) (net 3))
 (segment (start 26.352001 34.272001) (end 26.472001 34.272001) (width 0.6) (layer B.Cu) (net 3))
 (segment (start 13.05 30.995) (end 13.05 31.2) (width 0.4) (layer B.Cu) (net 3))
 (segment (start 14.025 30.02) (end 13.05 30.995) (width 0.4) (layer B.Cu) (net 3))
 (segment (start 22.1 30.02) (end 14.025 30.02) (width 0.6) (layer B.Cu) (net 3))
 (segment (start 36.65 8.74) (end 36.65 7.65) (width 0.6) (layer B.Cu) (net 3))
 (segment (start 33.216094 4.216094) (end 22.468124 4.216094) (width 0.6) (layer B.Cu) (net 3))
 (segment (start 21.608124 3.356094) (end 22.468124 4.216094) (width 0.4) (layer B.Cu) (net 3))
 (segment (start 36.65 7.65) (end 33.216094 4.216094) (width 0.6) (layer B.Cu) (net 3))
 (segment (start 13.418124 3.356094) (end 21.608124 3.356094) (width 0.6) (layer B.Cu) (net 3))
 (segment (start 23.302081 40.18) (end 22.1 40.18) (width 0.4) (layer B.Cu) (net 9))
 (segment (start 33.939762 40.18) (end 23.302081 40.18) (width 0.6) (layer B.Cu) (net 9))
 (segment (start 35.988001 38.131761) (end 33.939762 40.18) (width 0.6) (layer B.Cu) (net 9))
 (segment (start 35.988001 37.681999) (end 35.988001 38.131761) (width 0.6) (layer B.Cu) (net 9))
 (segment (start 36.75 36.92) (end 35.988001 37.681999) (width 0.6) (layer B.Cu) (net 9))
 (segment (start 22.1 40.18) (end 20.02 40.18) (width 0.4) (layer B.Cu) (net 9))
 (segment (start 17.281271 42.918729) (end 3.523066 42.918729) (width 0.6) (layer B.Cu) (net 9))
 (segment (start 20.02 40.18) (end 17.281271 42.918729) (width 0.6) (layer B.Cu) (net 9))
 (segment (start 36.65 13.82) (end 23.024218 13.82) (width 0.6) (layer B.Cu) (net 9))
 (segment (start 19.388124 17.456094) (end 22.468124 14.376094) (width 0.6) (layer B.Cu) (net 9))
 (segment (start 3.468124 17.456094) (end 19.388124 17.456094) (width 0.6) (layer B.Cu) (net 9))
 (segment (start 23.024218 13.82) (end 22.468124 14.376094) (width 0.4) (layer B.Cu) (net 9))
 (segment (start 22.65 38.19) (end 22.1 37.64) (width 0.4) (layer B.Cu) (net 10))
 (segment (start 34.21 38.19) (end 22.65 38.19) (width 0.6) (layer B.Cu) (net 10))
 (segment (start 6.1 41.1) (end 5.378729 40.378729) (width 0.6) (layer B.Cu) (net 10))
 (segment (start 17.1 41.1) (end 6.1 41.1) (width 0.6) (layer B.Cu) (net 10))
 (segment (start 5.378729 40.378729) (end 3.523066 40.378729) (width 0.6) (layer B.Cu) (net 10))
 (segment (start 22.1 37.64) (end 20.56 37.64) (width 0.4) (layer B.Cu) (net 10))
 (segment (start 20.56 37.64) (end 17.1 41.1) (width 0.6) (layer B.Cu) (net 10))
 (segment (start 3.468124 19.996094) (end 19.388124 19.996094) (width 0.6) (layer B.Cu) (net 10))
 (segment (start 32.283906 16.916094) (end 34.11 15.09) (width 0.6) (layer B.Cu) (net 10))
 (segment (start 22.468124 16.916094) (end 32.283906 16.916094) (width 0.6) (layer B.Cu) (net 10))
 (segment (start 19.388124 19.996094) (end 22.468124 16.916094) (width 0.6) (layer B.Cu) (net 10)))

